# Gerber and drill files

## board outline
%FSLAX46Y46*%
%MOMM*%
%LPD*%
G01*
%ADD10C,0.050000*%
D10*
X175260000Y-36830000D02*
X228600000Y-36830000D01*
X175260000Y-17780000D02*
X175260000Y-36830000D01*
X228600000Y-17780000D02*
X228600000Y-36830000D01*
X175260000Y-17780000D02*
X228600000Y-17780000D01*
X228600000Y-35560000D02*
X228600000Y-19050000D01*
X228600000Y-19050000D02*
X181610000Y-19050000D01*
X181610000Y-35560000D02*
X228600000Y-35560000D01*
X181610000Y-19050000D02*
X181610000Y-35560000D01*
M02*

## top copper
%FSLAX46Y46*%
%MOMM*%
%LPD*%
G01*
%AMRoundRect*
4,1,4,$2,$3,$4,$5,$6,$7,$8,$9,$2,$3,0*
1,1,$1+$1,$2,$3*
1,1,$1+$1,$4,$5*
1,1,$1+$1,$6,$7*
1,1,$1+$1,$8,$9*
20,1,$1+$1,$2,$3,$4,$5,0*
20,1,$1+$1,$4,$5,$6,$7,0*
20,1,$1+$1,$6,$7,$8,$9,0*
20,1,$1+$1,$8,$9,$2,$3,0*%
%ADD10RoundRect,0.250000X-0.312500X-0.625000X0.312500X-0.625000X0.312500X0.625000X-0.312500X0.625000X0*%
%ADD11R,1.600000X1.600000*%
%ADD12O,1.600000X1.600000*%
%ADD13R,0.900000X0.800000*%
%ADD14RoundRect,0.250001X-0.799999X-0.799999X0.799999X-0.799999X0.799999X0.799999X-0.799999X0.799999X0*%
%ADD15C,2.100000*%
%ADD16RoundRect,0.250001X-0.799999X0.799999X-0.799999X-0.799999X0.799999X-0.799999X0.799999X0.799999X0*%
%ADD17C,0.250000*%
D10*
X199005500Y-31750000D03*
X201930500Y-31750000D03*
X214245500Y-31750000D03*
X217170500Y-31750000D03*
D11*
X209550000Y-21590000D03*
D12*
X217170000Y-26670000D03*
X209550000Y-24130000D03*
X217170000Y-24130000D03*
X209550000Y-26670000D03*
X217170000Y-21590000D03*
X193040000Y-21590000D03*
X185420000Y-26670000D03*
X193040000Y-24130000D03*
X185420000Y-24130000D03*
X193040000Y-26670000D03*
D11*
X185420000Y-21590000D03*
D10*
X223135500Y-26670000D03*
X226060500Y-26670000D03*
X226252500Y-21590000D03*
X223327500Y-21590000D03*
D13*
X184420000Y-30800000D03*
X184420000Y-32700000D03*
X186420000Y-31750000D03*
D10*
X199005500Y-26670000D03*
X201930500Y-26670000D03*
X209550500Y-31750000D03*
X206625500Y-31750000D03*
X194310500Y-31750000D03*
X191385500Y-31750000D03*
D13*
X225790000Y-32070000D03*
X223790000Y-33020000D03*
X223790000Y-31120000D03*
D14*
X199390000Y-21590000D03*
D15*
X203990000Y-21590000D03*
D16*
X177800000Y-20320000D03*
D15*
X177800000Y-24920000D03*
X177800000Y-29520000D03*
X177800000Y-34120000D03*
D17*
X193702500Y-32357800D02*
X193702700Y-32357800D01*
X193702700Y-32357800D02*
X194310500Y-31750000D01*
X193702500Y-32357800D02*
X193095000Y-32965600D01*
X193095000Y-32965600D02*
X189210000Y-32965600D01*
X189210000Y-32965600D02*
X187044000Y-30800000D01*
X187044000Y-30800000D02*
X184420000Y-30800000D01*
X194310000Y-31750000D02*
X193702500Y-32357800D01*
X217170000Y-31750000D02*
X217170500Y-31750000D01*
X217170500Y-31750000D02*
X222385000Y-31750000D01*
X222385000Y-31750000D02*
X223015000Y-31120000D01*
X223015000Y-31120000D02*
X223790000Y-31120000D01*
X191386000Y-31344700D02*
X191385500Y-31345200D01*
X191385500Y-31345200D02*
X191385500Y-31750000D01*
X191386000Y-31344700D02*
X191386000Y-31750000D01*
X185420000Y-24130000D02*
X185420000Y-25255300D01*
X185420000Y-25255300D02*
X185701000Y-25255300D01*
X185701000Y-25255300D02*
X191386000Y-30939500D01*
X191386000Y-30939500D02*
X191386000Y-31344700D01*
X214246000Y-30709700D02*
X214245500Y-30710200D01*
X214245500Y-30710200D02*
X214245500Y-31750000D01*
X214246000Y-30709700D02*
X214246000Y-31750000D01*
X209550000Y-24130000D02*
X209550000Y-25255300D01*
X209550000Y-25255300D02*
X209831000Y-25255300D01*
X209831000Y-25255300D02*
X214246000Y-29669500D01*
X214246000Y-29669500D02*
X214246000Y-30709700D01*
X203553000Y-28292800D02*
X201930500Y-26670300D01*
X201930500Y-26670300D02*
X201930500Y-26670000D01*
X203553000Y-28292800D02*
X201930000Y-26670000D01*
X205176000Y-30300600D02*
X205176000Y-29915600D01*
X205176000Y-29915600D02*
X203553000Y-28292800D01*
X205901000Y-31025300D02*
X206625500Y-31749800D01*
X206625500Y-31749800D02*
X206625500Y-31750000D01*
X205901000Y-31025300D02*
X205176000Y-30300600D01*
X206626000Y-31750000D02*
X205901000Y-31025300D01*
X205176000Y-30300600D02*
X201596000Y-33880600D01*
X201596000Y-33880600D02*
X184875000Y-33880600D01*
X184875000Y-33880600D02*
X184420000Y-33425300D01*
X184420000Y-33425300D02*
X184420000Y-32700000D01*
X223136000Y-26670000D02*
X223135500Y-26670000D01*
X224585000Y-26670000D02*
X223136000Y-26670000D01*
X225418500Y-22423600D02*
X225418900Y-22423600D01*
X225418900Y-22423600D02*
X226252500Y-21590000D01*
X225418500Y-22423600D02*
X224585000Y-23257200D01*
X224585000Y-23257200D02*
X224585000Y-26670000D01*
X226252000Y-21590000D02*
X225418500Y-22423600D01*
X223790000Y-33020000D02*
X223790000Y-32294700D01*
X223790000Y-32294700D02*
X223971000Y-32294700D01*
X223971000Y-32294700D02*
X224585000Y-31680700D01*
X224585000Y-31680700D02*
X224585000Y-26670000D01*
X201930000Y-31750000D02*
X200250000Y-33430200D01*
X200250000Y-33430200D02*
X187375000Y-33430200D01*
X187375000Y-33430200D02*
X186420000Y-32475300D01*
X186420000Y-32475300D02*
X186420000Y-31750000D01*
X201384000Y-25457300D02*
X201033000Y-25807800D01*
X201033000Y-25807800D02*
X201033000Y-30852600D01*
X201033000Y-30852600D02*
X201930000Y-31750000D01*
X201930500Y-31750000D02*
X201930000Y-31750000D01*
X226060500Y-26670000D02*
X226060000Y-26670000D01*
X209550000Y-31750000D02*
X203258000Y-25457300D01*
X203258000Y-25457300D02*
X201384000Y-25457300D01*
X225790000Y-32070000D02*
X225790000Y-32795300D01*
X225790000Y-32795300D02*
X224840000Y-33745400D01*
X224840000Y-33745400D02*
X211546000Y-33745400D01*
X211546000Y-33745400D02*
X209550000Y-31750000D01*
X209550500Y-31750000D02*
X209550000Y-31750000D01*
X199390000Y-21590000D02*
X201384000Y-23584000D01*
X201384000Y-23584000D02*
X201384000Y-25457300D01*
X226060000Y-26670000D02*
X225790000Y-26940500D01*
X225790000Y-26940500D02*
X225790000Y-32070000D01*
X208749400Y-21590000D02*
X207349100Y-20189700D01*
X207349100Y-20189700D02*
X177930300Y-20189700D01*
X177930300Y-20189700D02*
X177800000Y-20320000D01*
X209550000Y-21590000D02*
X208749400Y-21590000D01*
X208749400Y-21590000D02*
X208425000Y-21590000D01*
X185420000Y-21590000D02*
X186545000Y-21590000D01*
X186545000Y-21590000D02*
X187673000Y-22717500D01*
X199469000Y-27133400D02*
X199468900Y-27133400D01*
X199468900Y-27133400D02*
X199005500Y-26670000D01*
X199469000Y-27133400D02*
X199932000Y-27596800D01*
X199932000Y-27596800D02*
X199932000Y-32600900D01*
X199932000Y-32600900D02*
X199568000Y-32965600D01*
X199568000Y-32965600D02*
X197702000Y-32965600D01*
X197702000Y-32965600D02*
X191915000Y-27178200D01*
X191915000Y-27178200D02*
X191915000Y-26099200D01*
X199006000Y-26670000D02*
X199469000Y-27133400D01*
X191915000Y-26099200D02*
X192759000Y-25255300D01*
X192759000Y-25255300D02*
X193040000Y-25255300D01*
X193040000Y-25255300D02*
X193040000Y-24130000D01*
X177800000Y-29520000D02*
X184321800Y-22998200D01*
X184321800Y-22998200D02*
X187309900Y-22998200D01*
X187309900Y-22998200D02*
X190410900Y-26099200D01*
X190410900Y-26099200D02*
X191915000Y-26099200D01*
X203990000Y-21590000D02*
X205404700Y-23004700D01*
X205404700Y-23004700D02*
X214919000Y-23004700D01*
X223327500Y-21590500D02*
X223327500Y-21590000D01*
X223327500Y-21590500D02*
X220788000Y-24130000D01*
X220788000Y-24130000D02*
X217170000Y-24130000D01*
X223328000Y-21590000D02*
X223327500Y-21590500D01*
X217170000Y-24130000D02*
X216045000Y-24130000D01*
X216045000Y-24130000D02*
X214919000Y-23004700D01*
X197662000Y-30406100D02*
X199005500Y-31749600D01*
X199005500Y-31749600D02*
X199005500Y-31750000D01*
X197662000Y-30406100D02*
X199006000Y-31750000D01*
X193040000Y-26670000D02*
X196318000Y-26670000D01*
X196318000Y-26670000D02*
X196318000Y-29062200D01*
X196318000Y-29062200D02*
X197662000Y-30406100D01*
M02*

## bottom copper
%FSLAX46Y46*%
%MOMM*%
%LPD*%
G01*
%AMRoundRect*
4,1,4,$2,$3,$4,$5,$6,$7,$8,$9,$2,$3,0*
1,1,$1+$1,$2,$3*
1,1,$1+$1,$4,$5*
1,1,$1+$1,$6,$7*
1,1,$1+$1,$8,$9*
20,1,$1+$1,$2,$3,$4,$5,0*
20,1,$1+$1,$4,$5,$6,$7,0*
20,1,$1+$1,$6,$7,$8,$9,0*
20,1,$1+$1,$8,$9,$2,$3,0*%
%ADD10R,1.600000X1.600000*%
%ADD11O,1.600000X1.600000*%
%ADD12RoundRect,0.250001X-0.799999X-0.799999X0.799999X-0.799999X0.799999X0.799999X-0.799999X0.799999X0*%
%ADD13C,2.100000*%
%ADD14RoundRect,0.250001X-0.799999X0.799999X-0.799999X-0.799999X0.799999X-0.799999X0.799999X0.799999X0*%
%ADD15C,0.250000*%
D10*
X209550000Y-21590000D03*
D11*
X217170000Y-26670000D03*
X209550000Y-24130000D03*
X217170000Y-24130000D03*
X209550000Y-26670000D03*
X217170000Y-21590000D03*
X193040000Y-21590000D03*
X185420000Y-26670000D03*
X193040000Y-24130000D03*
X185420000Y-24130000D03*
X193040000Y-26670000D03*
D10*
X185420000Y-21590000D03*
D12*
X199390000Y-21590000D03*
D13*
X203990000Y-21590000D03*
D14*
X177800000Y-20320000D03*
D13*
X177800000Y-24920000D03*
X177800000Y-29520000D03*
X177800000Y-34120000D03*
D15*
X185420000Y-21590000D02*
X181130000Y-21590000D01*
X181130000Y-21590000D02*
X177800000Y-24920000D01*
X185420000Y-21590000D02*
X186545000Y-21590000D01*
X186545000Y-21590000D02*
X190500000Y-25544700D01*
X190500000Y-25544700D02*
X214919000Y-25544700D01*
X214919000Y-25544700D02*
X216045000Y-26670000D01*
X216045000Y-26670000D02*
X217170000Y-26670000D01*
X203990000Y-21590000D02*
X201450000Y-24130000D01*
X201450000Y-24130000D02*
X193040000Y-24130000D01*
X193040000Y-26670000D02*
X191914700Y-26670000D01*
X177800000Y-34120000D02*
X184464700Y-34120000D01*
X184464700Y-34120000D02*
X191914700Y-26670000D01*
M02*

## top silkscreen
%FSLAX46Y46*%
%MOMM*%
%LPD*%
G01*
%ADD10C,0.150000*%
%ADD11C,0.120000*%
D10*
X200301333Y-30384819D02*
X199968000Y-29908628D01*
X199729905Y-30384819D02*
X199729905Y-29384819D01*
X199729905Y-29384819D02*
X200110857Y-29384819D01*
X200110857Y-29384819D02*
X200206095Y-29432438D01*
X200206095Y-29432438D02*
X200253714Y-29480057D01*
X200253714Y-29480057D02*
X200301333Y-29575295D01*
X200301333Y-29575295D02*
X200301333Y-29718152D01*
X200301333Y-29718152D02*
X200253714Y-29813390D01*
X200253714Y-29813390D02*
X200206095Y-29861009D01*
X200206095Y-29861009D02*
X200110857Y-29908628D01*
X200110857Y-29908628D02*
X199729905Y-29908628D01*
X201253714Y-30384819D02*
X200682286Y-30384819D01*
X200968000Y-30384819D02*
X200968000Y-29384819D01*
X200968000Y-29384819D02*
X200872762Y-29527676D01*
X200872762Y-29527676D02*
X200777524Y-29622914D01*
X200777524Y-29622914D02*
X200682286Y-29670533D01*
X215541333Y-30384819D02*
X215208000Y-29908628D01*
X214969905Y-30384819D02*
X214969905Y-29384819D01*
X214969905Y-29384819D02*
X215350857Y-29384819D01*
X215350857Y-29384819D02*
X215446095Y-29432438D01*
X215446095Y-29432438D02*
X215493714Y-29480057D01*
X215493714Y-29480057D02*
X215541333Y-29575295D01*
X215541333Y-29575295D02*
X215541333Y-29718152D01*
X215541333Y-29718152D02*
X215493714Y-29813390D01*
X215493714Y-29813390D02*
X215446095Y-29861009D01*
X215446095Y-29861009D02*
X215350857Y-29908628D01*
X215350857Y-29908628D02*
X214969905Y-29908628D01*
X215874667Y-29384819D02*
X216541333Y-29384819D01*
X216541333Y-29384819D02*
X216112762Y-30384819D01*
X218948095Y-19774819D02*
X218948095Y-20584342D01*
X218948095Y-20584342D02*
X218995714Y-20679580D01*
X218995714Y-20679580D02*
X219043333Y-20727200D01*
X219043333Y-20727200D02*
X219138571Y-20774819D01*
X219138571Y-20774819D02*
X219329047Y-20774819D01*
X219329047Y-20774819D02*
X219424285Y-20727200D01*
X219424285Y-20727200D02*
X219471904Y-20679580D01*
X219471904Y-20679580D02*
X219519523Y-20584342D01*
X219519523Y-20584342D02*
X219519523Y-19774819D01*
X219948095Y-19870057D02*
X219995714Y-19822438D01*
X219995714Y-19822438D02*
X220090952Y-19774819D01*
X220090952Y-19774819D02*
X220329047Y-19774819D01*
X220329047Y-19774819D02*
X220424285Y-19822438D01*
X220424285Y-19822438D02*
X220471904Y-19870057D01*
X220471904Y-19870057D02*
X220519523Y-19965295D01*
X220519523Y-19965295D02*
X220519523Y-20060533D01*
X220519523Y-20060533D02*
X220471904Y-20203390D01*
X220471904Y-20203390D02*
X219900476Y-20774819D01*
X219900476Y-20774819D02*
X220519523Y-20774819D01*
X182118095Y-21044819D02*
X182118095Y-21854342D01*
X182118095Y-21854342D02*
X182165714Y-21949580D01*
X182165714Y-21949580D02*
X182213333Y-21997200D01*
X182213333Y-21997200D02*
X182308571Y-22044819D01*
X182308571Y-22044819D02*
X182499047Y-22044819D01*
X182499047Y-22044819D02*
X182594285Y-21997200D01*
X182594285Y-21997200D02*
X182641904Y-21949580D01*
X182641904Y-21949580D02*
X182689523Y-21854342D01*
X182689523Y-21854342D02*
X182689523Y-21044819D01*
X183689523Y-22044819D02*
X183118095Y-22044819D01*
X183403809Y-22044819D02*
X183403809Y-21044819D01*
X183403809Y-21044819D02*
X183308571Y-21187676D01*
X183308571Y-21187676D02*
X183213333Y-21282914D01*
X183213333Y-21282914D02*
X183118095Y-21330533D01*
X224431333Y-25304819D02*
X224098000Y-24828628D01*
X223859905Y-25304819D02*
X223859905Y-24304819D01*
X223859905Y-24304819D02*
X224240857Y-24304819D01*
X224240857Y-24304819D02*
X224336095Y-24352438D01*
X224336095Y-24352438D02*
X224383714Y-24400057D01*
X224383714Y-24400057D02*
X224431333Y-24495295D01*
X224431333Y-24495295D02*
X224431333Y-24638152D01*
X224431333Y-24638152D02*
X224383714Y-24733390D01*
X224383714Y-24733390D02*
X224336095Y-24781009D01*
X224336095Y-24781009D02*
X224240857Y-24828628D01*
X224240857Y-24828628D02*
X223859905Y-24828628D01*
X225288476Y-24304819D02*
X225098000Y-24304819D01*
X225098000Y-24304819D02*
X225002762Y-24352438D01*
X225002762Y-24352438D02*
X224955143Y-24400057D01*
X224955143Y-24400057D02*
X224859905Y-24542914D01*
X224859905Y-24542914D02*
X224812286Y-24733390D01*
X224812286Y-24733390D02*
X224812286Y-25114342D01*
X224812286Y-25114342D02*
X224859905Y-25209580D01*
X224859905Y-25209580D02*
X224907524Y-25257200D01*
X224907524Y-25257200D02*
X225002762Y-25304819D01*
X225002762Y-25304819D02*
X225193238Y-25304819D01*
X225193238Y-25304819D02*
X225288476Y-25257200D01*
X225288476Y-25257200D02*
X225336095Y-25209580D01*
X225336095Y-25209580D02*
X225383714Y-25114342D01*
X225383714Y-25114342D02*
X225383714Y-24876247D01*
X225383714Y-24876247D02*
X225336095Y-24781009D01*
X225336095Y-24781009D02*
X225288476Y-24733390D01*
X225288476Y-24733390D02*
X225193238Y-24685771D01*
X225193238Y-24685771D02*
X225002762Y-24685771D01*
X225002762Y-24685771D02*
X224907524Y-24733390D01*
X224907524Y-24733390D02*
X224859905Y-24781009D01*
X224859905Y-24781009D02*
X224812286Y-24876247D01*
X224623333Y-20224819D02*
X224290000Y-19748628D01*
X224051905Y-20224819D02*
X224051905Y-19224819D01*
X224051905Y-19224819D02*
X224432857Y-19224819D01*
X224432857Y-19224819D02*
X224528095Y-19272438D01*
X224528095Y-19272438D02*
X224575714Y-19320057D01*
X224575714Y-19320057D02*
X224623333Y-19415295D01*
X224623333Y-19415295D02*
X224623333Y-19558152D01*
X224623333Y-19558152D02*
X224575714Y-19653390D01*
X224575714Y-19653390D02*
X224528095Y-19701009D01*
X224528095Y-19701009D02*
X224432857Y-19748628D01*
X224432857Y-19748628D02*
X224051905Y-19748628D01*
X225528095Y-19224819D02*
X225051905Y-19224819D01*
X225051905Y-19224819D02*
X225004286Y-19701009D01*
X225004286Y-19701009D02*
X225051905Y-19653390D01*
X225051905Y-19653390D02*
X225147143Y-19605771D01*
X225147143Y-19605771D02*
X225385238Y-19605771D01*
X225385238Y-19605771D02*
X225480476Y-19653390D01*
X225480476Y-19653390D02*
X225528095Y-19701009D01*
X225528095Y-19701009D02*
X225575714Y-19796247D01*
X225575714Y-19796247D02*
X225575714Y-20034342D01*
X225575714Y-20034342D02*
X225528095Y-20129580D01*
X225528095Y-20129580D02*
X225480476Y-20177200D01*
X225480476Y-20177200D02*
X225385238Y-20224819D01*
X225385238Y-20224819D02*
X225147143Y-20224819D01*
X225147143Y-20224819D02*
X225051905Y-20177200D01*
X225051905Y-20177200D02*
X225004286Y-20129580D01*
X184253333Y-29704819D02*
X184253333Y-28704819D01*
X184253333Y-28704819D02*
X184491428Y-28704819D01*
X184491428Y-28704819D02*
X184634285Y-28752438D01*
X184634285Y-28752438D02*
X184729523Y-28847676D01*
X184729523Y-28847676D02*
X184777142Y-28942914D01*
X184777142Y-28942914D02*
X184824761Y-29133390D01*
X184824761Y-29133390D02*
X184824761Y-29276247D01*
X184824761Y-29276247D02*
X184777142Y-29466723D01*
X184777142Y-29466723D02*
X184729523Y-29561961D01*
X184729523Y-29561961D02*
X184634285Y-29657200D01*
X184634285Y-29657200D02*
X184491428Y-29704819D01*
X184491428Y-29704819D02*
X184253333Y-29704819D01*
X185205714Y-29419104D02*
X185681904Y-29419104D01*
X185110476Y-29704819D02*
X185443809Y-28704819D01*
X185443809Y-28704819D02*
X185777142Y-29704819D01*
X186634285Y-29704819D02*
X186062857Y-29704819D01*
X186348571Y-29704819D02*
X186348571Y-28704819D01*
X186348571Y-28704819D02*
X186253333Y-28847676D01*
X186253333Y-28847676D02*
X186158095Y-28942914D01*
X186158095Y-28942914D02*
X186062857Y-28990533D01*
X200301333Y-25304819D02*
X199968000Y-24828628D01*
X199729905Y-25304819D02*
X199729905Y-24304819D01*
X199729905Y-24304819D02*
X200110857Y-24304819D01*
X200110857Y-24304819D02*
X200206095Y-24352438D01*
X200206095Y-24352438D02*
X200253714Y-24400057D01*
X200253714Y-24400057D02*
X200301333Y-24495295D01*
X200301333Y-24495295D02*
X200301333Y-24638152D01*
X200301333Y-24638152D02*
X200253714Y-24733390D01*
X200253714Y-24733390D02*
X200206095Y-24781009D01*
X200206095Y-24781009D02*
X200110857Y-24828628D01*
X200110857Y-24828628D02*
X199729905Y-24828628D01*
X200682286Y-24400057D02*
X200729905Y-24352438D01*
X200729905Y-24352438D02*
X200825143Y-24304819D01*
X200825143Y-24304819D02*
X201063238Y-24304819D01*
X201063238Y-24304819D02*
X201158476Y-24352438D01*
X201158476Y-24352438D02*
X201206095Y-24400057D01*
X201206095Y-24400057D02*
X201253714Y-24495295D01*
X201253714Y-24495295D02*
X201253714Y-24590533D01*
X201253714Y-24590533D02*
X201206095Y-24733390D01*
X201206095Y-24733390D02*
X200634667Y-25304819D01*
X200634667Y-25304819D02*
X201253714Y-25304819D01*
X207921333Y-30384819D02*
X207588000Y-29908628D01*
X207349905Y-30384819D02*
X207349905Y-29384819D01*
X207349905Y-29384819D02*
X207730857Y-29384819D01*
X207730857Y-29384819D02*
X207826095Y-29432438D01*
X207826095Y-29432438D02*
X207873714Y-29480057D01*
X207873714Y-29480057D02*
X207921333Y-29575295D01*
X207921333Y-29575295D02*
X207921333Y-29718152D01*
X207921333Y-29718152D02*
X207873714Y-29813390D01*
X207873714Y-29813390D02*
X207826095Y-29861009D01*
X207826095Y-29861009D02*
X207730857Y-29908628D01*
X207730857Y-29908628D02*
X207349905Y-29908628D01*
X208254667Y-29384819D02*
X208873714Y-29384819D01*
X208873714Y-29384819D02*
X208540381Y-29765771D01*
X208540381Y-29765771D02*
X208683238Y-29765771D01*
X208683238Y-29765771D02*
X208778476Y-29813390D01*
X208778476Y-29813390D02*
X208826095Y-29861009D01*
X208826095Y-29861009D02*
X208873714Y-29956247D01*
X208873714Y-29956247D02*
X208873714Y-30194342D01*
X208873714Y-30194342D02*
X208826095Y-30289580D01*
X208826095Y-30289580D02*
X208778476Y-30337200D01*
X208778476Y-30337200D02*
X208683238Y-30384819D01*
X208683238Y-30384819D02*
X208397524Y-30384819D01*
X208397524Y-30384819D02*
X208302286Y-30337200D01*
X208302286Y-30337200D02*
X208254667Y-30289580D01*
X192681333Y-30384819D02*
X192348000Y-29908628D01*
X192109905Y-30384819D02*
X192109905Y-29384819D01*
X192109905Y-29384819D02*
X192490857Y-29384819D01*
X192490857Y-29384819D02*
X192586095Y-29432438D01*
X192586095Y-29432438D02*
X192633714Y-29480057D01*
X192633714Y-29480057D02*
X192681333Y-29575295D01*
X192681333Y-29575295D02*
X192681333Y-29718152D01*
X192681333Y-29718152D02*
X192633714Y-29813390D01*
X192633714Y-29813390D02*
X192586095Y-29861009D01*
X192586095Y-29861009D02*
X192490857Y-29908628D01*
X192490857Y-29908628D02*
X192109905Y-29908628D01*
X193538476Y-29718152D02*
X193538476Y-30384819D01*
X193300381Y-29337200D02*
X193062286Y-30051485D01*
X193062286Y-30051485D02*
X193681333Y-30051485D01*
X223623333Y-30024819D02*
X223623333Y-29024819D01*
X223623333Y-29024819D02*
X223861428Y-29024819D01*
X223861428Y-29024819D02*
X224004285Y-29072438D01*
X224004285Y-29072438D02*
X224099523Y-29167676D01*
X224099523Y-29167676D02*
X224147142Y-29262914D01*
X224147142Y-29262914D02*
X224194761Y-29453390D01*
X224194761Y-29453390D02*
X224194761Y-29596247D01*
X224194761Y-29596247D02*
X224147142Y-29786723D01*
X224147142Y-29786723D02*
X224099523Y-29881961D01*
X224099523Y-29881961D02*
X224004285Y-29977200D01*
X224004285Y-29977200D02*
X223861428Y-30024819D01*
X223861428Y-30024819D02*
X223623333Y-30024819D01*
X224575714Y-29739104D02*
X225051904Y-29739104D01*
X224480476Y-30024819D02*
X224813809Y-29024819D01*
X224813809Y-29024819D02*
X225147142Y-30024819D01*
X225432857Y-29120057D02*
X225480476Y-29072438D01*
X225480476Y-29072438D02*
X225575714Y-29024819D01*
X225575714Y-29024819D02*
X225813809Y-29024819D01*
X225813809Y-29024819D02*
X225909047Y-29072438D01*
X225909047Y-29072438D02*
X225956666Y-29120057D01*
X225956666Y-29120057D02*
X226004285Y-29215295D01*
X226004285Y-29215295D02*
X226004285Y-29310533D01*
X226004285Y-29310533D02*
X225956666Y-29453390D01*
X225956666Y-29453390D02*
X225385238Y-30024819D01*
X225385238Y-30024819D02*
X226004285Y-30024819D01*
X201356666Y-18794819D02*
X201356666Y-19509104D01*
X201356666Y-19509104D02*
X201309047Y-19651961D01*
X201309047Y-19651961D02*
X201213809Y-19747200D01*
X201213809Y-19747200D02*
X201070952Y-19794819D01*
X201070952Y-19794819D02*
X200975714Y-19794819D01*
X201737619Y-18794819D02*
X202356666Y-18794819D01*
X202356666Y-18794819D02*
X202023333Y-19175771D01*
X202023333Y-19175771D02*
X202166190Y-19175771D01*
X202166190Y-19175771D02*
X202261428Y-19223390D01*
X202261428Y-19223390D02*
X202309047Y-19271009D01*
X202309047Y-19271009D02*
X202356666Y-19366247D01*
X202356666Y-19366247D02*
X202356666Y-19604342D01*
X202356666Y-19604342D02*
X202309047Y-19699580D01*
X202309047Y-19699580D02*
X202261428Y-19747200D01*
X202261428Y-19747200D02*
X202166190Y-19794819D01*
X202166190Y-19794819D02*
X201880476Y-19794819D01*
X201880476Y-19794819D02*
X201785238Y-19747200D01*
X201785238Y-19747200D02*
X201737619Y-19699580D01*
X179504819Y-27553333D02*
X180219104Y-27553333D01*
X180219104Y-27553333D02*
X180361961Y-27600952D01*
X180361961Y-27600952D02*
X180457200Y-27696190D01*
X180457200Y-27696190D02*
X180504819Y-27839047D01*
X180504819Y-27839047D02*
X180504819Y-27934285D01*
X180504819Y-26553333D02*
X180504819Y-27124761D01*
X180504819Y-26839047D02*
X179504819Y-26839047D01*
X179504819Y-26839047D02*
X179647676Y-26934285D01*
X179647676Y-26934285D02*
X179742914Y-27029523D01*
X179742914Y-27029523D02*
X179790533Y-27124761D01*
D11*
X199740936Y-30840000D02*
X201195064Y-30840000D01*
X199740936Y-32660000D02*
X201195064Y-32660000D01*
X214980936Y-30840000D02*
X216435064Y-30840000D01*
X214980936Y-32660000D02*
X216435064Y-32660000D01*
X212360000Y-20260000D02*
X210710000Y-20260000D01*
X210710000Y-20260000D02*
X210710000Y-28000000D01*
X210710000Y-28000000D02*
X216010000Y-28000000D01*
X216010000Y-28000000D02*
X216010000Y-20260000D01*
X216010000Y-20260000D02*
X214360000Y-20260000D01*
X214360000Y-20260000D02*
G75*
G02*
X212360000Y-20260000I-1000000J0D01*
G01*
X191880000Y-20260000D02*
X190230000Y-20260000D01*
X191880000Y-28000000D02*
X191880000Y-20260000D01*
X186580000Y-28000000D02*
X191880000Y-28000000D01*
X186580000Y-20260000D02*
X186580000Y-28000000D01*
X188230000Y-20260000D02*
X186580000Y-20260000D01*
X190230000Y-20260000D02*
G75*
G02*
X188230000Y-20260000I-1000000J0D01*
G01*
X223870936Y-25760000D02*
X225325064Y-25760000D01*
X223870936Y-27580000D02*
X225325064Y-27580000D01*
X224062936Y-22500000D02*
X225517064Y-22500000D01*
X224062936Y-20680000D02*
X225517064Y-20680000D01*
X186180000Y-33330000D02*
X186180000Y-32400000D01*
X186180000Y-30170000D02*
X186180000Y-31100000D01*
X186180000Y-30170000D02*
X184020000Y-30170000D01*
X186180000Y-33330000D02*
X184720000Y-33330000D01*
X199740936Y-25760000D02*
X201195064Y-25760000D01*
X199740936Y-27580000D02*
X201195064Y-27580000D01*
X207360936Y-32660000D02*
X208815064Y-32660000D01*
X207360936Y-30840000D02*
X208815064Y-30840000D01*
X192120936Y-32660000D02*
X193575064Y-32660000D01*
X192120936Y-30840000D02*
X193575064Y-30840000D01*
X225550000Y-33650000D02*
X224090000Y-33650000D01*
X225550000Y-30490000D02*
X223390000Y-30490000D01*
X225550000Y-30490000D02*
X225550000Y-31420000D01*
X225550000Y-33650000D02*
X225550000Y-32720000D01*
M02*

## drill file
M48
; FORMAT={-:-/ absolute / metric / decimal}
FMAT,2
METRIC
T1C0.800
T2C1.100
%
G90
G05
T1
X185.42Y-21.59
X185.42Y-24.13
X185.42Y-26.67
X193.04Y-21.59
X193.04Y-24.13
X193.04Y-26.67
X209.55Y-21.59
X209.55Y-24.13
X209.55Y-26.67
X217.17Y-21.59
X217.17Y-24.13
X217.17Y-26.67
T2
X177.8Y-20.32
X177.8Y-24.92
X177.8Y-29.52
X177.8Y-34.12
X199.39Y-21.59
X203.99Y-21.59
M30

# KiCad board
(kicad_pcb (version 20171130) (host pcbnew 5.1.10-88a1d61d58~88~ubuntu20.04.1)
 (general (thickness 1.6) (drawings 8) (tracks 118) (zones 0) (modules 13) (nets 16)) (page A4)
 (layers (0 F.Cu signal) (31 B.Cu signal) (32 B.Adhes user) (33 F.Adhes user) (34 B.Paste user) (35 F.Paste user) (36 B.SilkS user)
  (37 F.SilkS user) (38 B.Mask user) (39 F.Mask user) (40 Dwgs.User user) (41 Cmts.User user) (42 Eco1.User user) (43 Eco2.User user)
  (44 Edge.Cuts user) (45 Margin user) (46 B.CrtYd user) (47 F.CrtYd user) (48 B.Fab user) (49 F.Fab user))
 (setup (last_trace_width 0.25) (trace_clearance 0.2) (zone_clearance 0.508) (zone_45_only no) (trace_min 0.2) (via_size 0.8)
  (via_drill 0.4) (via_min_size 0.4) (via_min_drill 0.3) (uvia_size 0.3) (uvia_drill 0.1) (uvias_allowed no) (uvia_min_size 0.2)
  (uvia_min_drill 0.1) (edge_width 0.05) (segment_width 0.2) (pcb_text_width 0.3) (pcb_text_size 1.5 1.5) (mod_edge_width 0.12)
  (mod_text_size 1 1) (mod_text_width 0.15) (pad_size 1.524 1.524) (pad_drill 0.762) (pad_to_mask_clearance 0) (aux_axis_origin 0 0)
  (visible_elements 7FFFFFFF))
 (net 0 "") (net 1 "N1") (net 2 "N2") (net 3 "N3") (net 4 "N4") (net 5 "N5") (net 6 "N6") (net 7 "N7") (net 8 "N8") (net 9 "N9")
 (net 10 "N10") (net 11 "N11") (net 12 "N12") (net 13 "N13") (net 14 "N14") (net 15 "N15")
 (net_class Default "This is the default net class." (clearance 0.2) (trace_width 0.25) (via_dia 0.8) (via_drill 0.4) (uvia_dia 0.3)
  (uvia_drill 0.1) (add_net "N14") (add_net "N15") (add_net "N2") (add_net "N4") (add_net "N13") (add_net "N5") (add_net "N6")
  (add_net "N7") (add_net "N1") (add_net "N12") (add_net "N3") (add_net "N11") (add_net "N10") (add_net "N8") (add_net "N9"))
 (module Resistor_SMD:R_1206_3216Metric (layer F.Cu) (at 200.468 31.75)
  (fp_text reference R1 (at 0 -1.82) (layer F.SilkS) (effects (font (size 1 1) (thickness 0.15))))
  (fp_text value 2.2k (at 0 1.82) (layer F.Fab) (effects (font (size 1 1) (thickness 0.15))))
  (fp_line (start -0.727064 -0.91) (end 0.727064 -0.91) (layer F.SilkS) (width 0.12))
  (fp_line (start -0.727064 0.91) (end 0.727064 0.91) (layer F.SilkS) (width 0.12))
  (pad 1 smd roundrect (at -1.4625 0) (size 1.125 1.75) (layers F.Cu F.Paste F.Mask) (roundrect_rratio 0.222222) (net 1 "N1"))
  (pad 2 smd roundrect (at 1.4625 0) (size 1.125 1.75) (layers F.Cu F.Paste F.Mask) (roundrect_rratio 0.222222) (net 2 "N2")))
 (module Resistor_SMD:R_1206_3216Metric (layer F.Cu) (at 215.708 31.75)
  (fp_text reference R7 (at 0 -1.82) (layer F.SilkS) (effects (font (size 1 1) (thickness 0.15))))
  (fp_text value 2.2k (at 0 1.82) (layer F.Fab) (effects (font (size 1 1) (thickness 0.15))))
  (fp_line (start -0.727064 -0.91) (end 0.727064 -0.91) (layer F.SilkS) (width 0.12))
  (fp_line (start -0.727064 0.91) (end 0.727064 0.91) (layer F.SilkS) (width 0.12))
  (pad 1 smd roundrect (at -1.4625 0) (size 1.125 1.75) (layers F.Cu F.Paste F.Mask) (roundrect_rratio 0.222222) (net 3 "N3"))
  (pad 2 smd roundrect (at 1.4625 0) (size 1.125 1.75) (layers F.Cu F.Paste F.Mask) (roundrect_rratio 0.222222) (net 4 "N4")))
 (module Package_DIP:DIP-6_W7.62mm (layer F.Cu) (at 209.55 21.59)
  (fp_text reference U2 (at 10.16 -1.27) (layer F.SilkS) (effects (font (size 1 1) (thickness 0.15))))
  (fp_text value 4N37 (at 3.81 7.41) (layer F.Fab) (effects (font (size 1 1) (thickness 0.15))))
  (fp_line (start 2.81 -1.33) (end 1.16 -1.33) (layer F.SilkS) (width 0.12))
  (fp_line (start 1.16 -1.33) (end 1.16 6.41) (layer F.SilkS) (width 0.12))
  (fp_line (start 1.16 6.41) (end 6.46 6.41) (layer F.SilkS) (width 0.12))
  (fp_line (start 6.46 6.41) (end 6.46 -1.33) (layer F.SilkS) (width 0.12))
  (fp_line (start 6.46 -1.33) (end 4.81 -1.33) (layer F.SilkS) (width 0.12))
  (fp_arc (start 3.81 -1.33) (end 2.81 -1.33) (angle -180) (layer F.SilkS) (width 0.12))
  (pad 1 thru_hole rect (at 0 0) (size 1.6 1.6) (drill 0.8) (layers *.Cu *.Mask) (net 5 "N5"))
  (pad 4 thru_hole oval (at 7.62 5.08) (size 1.6 1.6) (drill 0.8) (layers *.Cu *.Mask) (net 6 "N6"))
  (pad 2 thru_hole oval (at 0 2.54) (size 1.6 1.6) (drill 0.8) (layers *.Cu *.Mask) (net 3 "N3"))
  (pad 5 thru_hole oval (at 7.62 2.54) (size 1.6 1.6) (drill 0.8) (layers *.Cu *.Mask) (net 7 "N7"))
  (pad 3 thru_hole oval (at 0 5.08) (size 1.6 1.6) (drill 0.8) (layers *.Cu *.Mask) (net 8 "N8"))
  (pad 6 thru_hole oval (at 7.62 0) (size 1.6 1.6) (drill 0.8) (layers *.Cu *.Mask) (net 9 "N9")))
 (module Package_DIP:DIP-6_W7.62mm (layer F.Cu) (at 185.42 21.59)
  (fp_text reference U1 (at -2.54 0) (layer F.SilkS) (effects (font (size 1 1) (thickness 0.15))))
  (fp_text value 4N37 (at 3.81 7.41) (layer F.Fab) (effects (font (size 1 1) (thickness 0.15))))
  (fp_line (start 6.46 -1.33) (end 4.81 -1.33) (layer F.SilkS) (width 0.12))
  (fp_line (start 6.46 6.41) (end 6.46 -1.33) (layer F.SilkS) (width 0.12))
  (fp_line (start 1.16 6.41) (end 6.46 6.41) (layer F.SilkS) (width 0.12))
  (fp_line (start 1.16 -1.33) (end 1.16 6.41) (layer F.SilkS) (width 0.12))
  (fp_line (start 2.81 -1.33) (end 1.16 -1.33) (layer F.SilkS) (width 0.12))
  (fp_arc (start 3.81 -1.33) (end 2.81 -1.33) (angle -180) (layer F.SilkS) (width 0.12))
  (pad 6 thru_hole oval (at 7.62 0) (size 1.6 1.6) (drill 0.8) (layers *.Cu *.Mask) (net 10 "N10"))
  (pad 3 thru_hole oval (at 0 5.08) (size 1.6 1.6) (drill 0.8) (layers *.Cu *.Mask) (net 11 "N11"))
  (pad 5 thru_hole oval (at 7.62 2.54) (size 1.6 1.6) (drill 0.8) (layers *.Cu *.Mask) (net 7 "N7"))
  (pad 2 thru_hole oval (at 0 2.54) (size 1.6 1.6) (drill 0.8) (layers *.Cu *.Mask) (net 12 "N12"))
  (pad 4 thru_hole oval (at 7.62 5.08) (size 1.6 1.6) (drill 0.8) (layers *.Cu *.Mask) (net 1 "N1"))
  (pad 1 thru_hole rect (at 0 0) (size 1.6 1.6) (drill 0.8) (layers *.Cu *.Mask) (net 6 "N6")))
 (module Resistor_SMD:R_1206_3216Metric (layer F.Cu) (at 224.598 26.67)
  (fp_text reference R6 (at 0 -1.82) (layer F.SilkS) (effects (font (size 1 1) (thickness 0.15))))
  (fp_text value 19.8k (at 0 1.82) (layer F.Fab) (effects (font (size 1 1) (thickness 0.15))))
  (fp_line (start -0.727064 -0.91) (end 0.727064 -0.91) (layer F.SilkS) (width 0.12))
  (fp_line (start -0.727064 0.91) (end 0.727064 0.91) (layer F.SilkS) (width 0.12))
  (pad 1 smd roundrect (at -1.4625 0) (size 1.125 1.75) (layers F.Cu F.Paste F.Mask) (roundrect_rratio 0.222222) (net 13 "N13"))
  (pad 2 smd roundrect (at 1.4625 0) (size 1.125 1.75) (layers F.Cu F.Paste F.Mask) (roundrect_rratio 0.222222) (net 2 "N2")))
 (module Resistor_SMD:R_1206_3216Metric (layer F.Cu) (at 224.79 21.59)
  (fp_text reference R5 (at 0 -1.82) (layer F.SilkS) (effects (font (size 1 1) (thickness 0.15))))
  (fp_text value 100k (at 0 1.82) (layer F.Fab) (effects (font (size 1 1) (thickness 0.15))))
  (fp_line (start -0.727064 0.91) (end 0.727064 0.91) (layer F.SilkS) (width 0.12))
  (fp_line (start -0.727064 -0.91) (end 0.727064 -0.91) (layer F.SilkS) (width 0.12))
  (pad 2 smd roundrect (at 1.4625 0) (size 1.125 1.75) (layers F.Cu F.Paste F.Mask) (roundrect_rratio 0.222222) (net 13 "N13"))
  (pad 1 smd roundrect (at -1.4625 0) (size 1.125 1.75) (layers F.Cu F.Paste F.Mask) (roundrect_rratio 0.222222) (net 7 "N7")))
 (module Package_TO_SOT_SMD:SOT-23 (layer F.Cu) (at 185.42 31.75)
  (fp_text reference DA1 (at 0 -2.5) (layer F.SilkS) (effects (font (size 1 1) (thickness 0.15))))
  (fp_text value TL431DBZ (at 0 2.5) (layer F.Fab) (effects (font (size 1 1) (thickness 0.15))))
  (fp_line (start 0.76 1.58) (end 0.76 0.65) (layer F.SilkS) (width 0.12))
  (fp_line (start 0.76 -1.58) (end 0.76 -0.65) (layer F.SilkS) (width 0.12))
  (fp_line (start 0.76 -1.58) (end -1.4 -1.58) (layer F.SilkS) (width 0.12))
  (fp_line (start 0.76 1.58) (end -0.7 1.58) (layer F.SilkS) (width 0.12))
  (pad 1 smd rect (at -1 -0.95) (size 0.9 0.8) (layers F.Cu F.Paste F.Mask) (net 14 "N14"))
  (pad 2 smd rect (at -1 0.95) (size 0.9 0.8) (layers F.Cu F.Paste F.Mask) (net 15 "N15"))
  (pad 3 smd rect (at 1 0) (size 0.9 0.8) (layers F.Cu F.Paste F.Mask) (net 2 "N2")))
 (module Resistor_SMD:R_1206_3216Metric (layer F.Cu) (at 200.468 26.67)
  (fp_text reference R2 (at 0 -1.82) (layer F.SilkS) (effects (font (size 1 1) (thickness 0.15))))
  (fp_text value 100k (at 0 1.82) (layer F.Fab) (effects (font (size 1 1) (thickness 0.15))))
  (fp_line (start -0.727064 -0.91) (end 0.727064 -0.91) (layer F.SilkS) (width 0.12))
  (fp_line (start -0.727064 0.91) (end 0.727064 0.91) (layer F.SilkS) (width 0.12))
  (pad 1 smd roundrect (at -1.4625 0) (size 1.125 1.75) (layers F.Cu F.Paste F.Mask) (roundrect_rratio 0.222222) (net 7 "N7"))
  (pad 2 smd roundrect (at 1.4625 0) (size 1.125 1.75) (layers F.Cu F.Paste F.Mask) (roundrect_rratio 0.222222) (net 15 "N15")))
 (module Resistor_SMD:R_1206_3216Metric (layer F.Cu) (at 208.088 31.75)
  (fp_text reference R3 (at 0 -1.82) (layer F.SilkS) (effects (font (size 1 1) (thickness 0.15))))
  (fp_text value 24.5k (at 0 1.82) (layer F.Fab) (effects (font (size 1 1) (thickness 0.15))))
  (fp_line (start -0.727064 0.91) (end 0.727064 0.91) (layer F.SilkS) (width 0.12))
  (fp_line (start -0.727064 -0.91) (end 0.727064 -0.91) (layer F.SilkS) (width 0.12))
  (pad 2 smd roundrect (at 1.4625 0) (size 1.125 1.75) (layers F.Cu F.Paste F.Mask) (roundrect_rratio 0.222222) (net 2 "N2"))
  (pad 1 smd roundrect (at -1.4625 0) (size 1.125 1.75) (layers F.Cu F.Paste F.Mask) (roundrect_rratio 0.222222) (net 15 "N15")))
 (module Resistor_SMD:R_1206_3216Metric (layer F.Cu) (at 192.848 31.75)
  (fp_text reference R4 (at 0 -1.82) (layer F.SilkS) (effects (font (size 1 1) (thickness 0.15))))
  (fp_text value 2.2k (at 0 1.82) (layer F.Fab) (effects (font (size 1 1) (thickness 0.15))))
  (fp_line (start -0.727064 0.91) (end 0.727064 0.91) (layer F.SilkS) (width 0.12))
  (fp_line (start -0.727064 -0.91) (end 0.727064 -0.91) (layer F.SilkS) (width 0.12))
  (pad 2 smd roundrect (at 1.4625 0) (size 1.125 1.75) (layers F.Cu F.Paste F.Mask) (roundrect_rratio 0.222222) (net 14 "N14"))
  (pad 1 smd roundrect (at -1.4625 0) (size 1.125 1.75) (layers F.Cu F.Paste F.Mask) (roundrect_rratio 0.222222) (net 12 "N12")))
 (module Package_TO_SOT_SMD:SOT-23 (layer F.Cu) (at 224.79 32.07)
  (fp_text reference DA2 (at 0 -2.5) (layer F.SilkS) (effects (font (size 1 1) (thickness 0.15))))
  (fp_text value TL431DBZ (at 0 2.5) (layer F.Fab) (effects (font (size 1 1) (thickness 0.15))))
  (fp_line (start 0.76 1.58) (end -0.7 1.58) (layer F.SilkS) (width 0.12))
  (fp_line (start 0.76 -1.58) (end -1.4 -1.58) (layer F.SilkS) (width 0.12))
  (fp_line (start 0.76 -1.58) (end 0.76 -0.65) (layer F.SilkS) (width 0.12))
  (fp_line (start 0.76 1.58) (end 0.76 0.65) (layer F.SilkS) (width 0.12))
  (pad 3 smd rect (at 1 0) (size 0.9 0.8) (layers F.Cu F.Paste F.Mask) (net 2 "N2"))
  (pad 2 smd rect (at -1 0.95) (size 0.9 0.8) (layers F.Cu F.Paste F.Mask) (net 13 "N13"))
  (pad 1 smd rect (at -1 -0.95) (size 0.9 0.8) (layers F.Cu F.Paste F.Mask) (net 4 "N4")))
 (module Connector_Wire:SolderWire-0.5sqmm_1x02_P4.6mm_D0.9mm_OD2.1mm (layer F.Cu) (at 199.39 21.59)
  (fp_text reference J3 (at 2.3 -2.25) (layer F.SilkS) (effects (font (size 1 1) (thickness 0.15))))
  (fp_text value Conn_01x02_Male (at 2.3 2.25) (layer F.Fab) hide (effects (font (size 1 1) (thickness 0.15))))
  (pad 1 thru_hole roundrect (at 0 0) (size 2.1 2.1) (drill 1.1) (layers *.Cu *.Mask) (roundrect_rratio 0.119048) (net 2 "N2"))
  (pad 2 thru_hole circle (at 4.6 0) (size 2.1 2.1) (drill 1.1) (layers *.Cu *.Mask) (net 7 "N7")))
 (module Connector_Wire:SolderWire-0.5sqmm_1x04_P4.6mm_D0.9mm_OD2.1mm (layer F.Cu) (at 177.8 20.32 270)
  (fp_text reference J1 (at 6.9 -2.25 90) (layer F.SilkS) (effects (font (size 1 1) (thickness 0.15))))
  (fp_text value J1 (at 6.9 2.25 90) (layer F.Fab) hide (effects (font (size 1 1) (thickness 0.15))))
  (pad 1 thru_hole roundrect (at 0 0 270) (size 2.1 2.1) (drill 1.1) (layers *.Cu *.Mask) (roundrect_rratio 0.119048) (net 5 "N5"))
  (pad 2 thru_hole circle (at 4.6 0 270) (size 2.1 2.1) (drill 1.1) (layers *.Cu *.Mask) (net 6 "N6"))
  (pad 3 thru_hole circle (at 9.2 0 270) (size 2.1 2.1) (drill 1.1) (layers *.Cu *.Mask) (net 7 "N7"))
  (pad 4 thru_hole circle (at 13.8 0 270) (size 2.1 2.1) (drill 1.1) (layers *.Cu *.Mask) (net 1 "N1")))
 (gr_line (start 175.26 36.83) (end 228.6 36.83) (layer Edge.Cuts) (width 0.05))
 (gr_line (start 175.26 17.78) (end 175.26 36.83) (layer Edge.Cuts) (width 0.05))
 (gr_line (start 228.6 17.78) (end 228.6 36.83) (layer Edge.Cuts) (width 0.05))
 (gr_line (start 175.26 17.78) (end 228.6 17.78) (layer Edge.Cuts) (width 0.05))
 (gr_line (start 228.6 35.56) (end 228.6 19.05) (layer Edge.Cuts) (width 0.05))
 (gr_line (start 228.6 19.05) (end 181.61 19.05) (layer Edge.Cuts) (width 0.05))
 (gr_line (start 181.61 35.56) (end 228.6 35.56) (layer Edge.Cuts) (width 0.05))
 (gr_line (start 181.61 19.05) (end 181.61 35.56) (layer Edge.Cuts) (width 0.05))
 (segment (start 193.7025 32.3578) (end 193.7027 32.3578) (width 0.25) (layer F.Cu) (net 14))
 (segment (start 193.7027 32.3578) (end 194.3105 31.75) (width 0.25) (layer F.Cu) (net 14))
 (segment (start 193.7025 32.3578) (end 193.095 32.9656) (width 0.25) (layer F.Cu) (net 14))
 (segment (start 193.095 32.9656) (end 189.21 32.9656) (width 0.25) (layer F.Cu) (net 14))
 (segment (start 189.21 32.9656) (end 187.044 30.8) (width 0.25) (layer F.Cu) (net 14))
 (segment (start 187.044 30.8) (end 184.42 30.8) (width 0.25) (layer F.Cu) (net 14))
 (segment (start 194.31 31.75) (end 193.7025 32.3578) (width 0.25) (layer F.Cu) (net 14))
 (segment (start 217.17 31.75) (end 217.1705 31.75) (width 0.25) (layer F.Cu) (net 4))
 (segment (start 217.1705 31.75) (end 222.385 31.75) (width 0.25) (layer F.Cu) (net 4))
 (segment (start 222.385 31.75) (end 223.015 31.12) (width 0.25) (layer F.Cu) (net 4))
 (segment (start 223.015 31.12) (end 223.79 31.12) (width 0.25) (layer F.Cu) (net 4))
 (segment (start 191.386 31.3447) (end 191.3855 31.3452) (width 0.25) (layer F.Cu) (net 12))
 (segment (start 191.3855 31.3452) (end 191.3855 31.75) (width 0.25) (layer F.Cu) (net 12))
 (segment (start 191.386 31.3447) (end 191.386 31.75) (width 0.25) (layer F.Cu) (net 12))
 (segment (start 185.42 24.13) (end 185.42 25.2553) (width 0.25) (layer F.Cu) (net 12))
 (segment (start 185.42 25.2553) (end 185.701 25.2553) (width 0.25) (layer F.Cu) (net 12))
 (segment (start 185.701 25.2553) (end 191.386 30.9395) (width 0.25) (layer F.Cu) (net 12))
 (segment (start 191.386 30.9395) (end 191.386 31.3447) (width 0.25) (layer F.Cu) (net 12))
 (segment (start 214.246 30.7097) (end 214.2455 30.7102) (width 0.25) (layer F.Cu) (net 3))
 (segment (start 214.2455 30.7102) (end 214.2455 31.75) (width 0.25) (layer F.Cu) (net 3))
 (segment (start 214.246 30.7097) (end 214.246 31.75) (width 0.25) (layer F.Cu) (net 3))
 (segment (start 209.55 24.13) (end 209.55 25.2553) (width 0.25) (layer F.Cu) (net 3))
 (segment (start 209.55 25.2553) (end 209.831 25.2553) (width 0.25) (layer F.Cu) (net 3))
 (segment (start 209.831 25.2553) (end 214.246 29.6695) (width 0.25) (layer F.Cu) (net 3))
 (segment (start 214.246 29.6695) (end 214.246 30.7097) (width 0.25) (layer F.Cu) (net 3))
 (segment (start 203.553 28.2928) (end 201.9305 26.6703) (width 0.25) (layer F.Cu) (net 15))
 (segment (start 201.9305 26.6703) (end 201.9305 26.67) (width 0.25) (layer F.Cu) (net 15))
 (segment (start 203.553 28.2928) (end 201.93 26.67) (width 0.25) (layer F.Cu) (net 15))
 (segment (start 205.176 30.3006) (end 205.176 29.9156) (width 0.25) (layer F.Cu) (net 15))
 (segment (start 205.176 29.9156) (end 203.553 28.2928) (width 0.25) (layer F.Cu) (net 15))
 (segment (start 205.901 31.0253) (end 206.6255 31.7498) (width 0.25) (layer F.Cu) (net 15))
 (segment (start 206.6255 31.7498) (end 206.6255 31.75) (width 0.25) (layer F.Cu) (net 15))
 (segment (start 205.901 31.0253) (end 205.176 30.3006) (width 0.25) (layer F.Cu) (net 15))
 (segment (start 206.626 31.75) (end 205.901 31.0253) (width 0.25) (layer F.Cu) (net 15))
 (segment (start 205.176 30.3006) (end 201.596 33.8806) (width 0.25) (layer F.Cu) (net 15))
 (segment (start 201.596 33.8806) (end 184.875 33.8806) (width 0.25) (layer F.Cu) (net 15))
 (segment (start 184.875 33.8806) (end 184.42 33.4253) (width 0.25) (layer F.Cu) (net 15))
 (segment (start 184.42 33.4253) (end 184.42 32.7) (width 0.25) (layer F.Cu) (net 15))
 (segment (start 223.136 26.67) (end 223.1355 26.67) (width 0.25) (layer F.Cu) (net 13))
 (segment (start 224.585 26.67) (end 223.136 26.67) (width 0.25) (layer F.Cu) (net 13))
 (segment (start 225.4185 22.4236) (end 225.4189 22.4236) (width 0.25) (layer F.Cu) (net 13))
 (segment (start 225.4189 22.4236) (end 226.2525 21.59) (width 0.25) (layer F.Cu) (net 13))
 (segment (start 225.4185 22.4236) (end 224.585 23.2572) (width 0.25) (layer F.Cu) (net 13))
 (segment (start 224.585 23.2572) (end 224.585 26.67) (width 0.25) (layer F.Cu) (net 13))
 (segment (start 226.252 21.59) (end 225.4185 22.4236) (width 0.25) (layer F.Cu) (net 13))
 (segment (start 223.79 33.02) (end 223.79 32.2947) (width 0.25) (layer F.Cu) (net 13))
 (segment (start 223.79 32.2947) (end 223.971 32.2947) (width 0.25) (layer F.Cu) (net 13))
 (segment (start 223.971 32.2947) (end 224.585 31.6807) (width 0.25) (layer F.Cu) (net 13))
 (segment (start 224.585 31.6807) (end 224.585 26.67) (width 0.25) (layer F.Cu) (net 13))
 (segment (start 201.93 31.75) (end 200.25 33.4302) (width 0.25) (layer F.Cu) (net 2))
 (segment (start 200.25 33.4302) (end 187.375 33.4302) (width 0.25) (layer F.Cu) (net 2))
 (segment (start 187.375 33.4302) (end 186.42 32.4753) (width 0.25) (layer F.Cu) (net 2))
 (segment (start 186.42 32.4753) (end 186.42 31.75) (width 0.25) (layer F.Cu) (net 2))
 (segment (start 201.384 25.4573) (end 201.033 25.8078) (width 0.25) (layer F.Cu) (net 2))
 (segment (start 201.033 25.8078) (end 201.033 30.8526) (width 0.25) (layer F.Cu) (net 2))
 (segment (start 201.033 30.8526) (end 201.93 31.75) (width 0.25) (layer F.Cu) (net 2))
 (segment (start 201.9305 31.75) (end 201.93 31.75) (width 0.25) (layer F.Cu) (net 2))
 (segment (start 226.0605 26.67) (end 226.06 26.67) (width 0.25) (layer F.Cu) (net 2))
 (segment (start 209.55 31.75) (end 203.258 25.4573) (width 0.25) (layer F.Cu) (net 2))
 (segment (start 203.258 25.4573) (end 201.384 25.4573) (width 0.25) (layer F.Cu) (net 2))
 (segment (start 225.79 32.07) (end 225.79 32.7953) (width 0.25) (layer F.Cu) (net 2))
 (segment (start 225.79 32.7953) (end 224.84 33.7454) (width 0.25) (layer F.Cu) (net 2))
 (segment (start 224.84 33.7454) (end 211.546 33.7454) (width 0.25) (layer F.Cu) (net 2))
 (segment (start 211.546 33.7454) (end 209.55 31.75) (width 0.25) (layer F.Cu) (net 2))
 (segment (start 209.5505 31.75) (end 209.55 31.75) (width 0.25) (layer F.Cu) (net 2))
 (segment (start 199.39 21.59) (end 201.384 23.584) (width 0.25) (layer F.Cu) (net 2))
 (segment (start 201.384 23.584) (end 201.384 25.4573) (width 0.25) (layer F.Cu) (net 2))
 (segment (start 226.06 26.67) (end 225.79 26.9405) (width 0.25) (layer F.Cu) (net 2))
 (segment (start 225.79 26.9405) (end 225.79 32.07) (width 0.25) (layer F.Cu) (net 2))
 (segment (start 208.7494 21.59) (end 207.3491 20.1897) (width 0.25) (layer F.Cu) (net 5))
 (segment (start 207.3491 20.1897) (end 177.9303 20.1897) (width 0.25) (layer F.Cu) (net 5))
 (segment (start 177.9303 20.1897) (end 177.8 20.32) (width 0.25) (layer F.Cu) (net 5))
 (segment (start 209.55 21.59) (end 208.7494 21.59) (width 0.25) (layer F.Cu) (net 5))
 (segment (start 208.7494 21.59) (end 208.425 21.59) (width 0.25) (layer F.Cu) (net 5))
 (segment (start 185.42 21.59) (end 181.13 21.59) (width 0.25) (layer B.Cu) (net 6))
 (segment (start 181.13 21.59) (end 177.8 24.92) (width 0.25) (layer B.Cu) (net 6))
 (segment (start 185.42 21.59) (end 186.545 21.59) (width 0.25) (layer B.Cu) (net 6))
 (segment (start 186.545 21.59) (end 190.5 25.5447) (width 0.25) (layer B.Cu) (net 6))
 (segment (start 190.5 25.5447) (end 214.919 25.5447) (width 0.25) (layer B.Cu) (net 6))
 (segment (start 214.919 25.5447) (end 216.045 26.67) (width 0.25) (layer B.Cu) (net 6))
 (segment (start 216.045 26.67) (end 217.17 26.67) (width 0.25) (layer B.Cu) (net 6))
 (segment (start 185.42 21.59) (end 186.545 21.59) (width 0.25) (layer F.Cu) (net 6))
 (segment (start 186.545 21.59) (end 187.673 22.7175) (width 0.25) (layer F.Cu) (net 6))
 (segment (start 199.469 27.1334) (end 199.4689 27.1334) (width 0.25) (layer F.Cu) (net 7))
 (segment (start 199.4689 27.1334) (end 199.0055 26.67) (width 0.25) (layer F.Cu) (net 7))
 (segment (start 199.469 27.1334) (end 199.932 27.5968) (width 0.25) (layer F.Cu) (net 7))
 (segment (start 199.932 27.5968) (end 199.932 32.6009) (width 0.25) (layer F.Cu) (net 7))
 (segment (start 199.932 32.6009) (end 199.568 32.9656) (width 0.25) (layer F.Cu) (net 7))
 (segment (start 199.568 32.9656) (end 197.702 32.9656) (width 0.25) (layer F.Cu) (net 7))
 (segment (start 197.702 32.9656) (end 191.915 27.1782) (width 0.25) (layer F.Cu) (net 7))
 (segment (start 191.915 27.1782) (end 191.915 26.0992) (width 0.25) (layer F.Cu) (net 7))
 (segment (start 199.006 26.67) (end 199.469 27.1334) (width 0.25) (layer F.Cu) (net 7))
 (segment (start 191.915 26.0992) (end 192.759 25.2553) (width 0.25) (layer F.Cu) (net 7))
 (segment (start 192.759 25.2553) (end 193.04 25.2553) (width 0.25) (layer F.Cu) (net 7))
 (segment (start 193.04 25.2553) (end 193.04 24.13) (width 0.25) (layer F.Cu) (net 7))
 (segment (start 177.8 29.52) (end 184.3218 22.9982) (width 0.25) (layer F.Cu) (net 7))
 (segment (start 184.3218 22.9982) (end 187.3099 22.9982) (width 0.25) (layer F.Cu) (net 7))
 (segment (start 187.3099 22.9982) (end 190.4109 26.0992) (width 0.25) (layer F.Cu) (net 7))
 (segment (start 190.4109 26.0992) (end 191.915 26.0992) (width 0.25) (layer F.Cu) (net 7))
 (segment (start 203.99 21.59) (end 201.45 24.13) (width 0.25) (layer B.Cu) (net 7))
 (segment (start 201.45 24.13) (end 193.04 24.13) (width 0.25) (layer B.Cu) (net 7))
 (segment (start 203.99 21.59) (end 205.4047 23.0047) (width 0.25) (layer F.Cu) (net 7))
 (segment (start 205.4047 23.0047) (end 214.919 23.0047) (width 0.25) (layer F.Cu) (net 7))
 (segment (start 223.3275 21.5905) (end 223.3275 21.59) (width 0.25) (layer F.Cu) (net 7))
 (segment (start 223.3275 21.5905) (end 220.788 24.13) (width 0.25) (layer F.Cu) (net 7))
 (segment (start 220.788 24.13) (end 217.17 24.13) (width 0.25) (layer F.Cu) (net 7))
 (segment (start 223.328 21.59) (end 223.3275 21.5905) (width 0.25) (layer F.Cu) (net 7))
 (segment (start 217.17 24.13) (end 216.045 24.13) (width 0.25) (layer F.Cu) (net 7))
 (segment (start 216.045 24.13) (end 214.919 23.0047) (width 0.25) (layer F.Cu) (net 7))
 (segment (start 193.04 26.67) (end 191.9147 26.67) (width 0.25) (layer B.Cu) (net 1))
 (segment (start 177.8 34.12) (end 184.4647 34.12) (width 0.25) (layer B.Cu) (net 1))
 (segment (start 184.4647 34.12) (end 191.9147 26.67) (width 0.25) (layer B.Cu) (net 1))
 (segment (start 197.662 30.4061) (end 199.0055 31.7496) (width 0.25) (layer F.Cu) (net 1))
 (segment (start 199.0055 31.7496) (end 199.0055 31.75) (width 0.25) (layer F.Cu) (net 1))
 (segment (start 197.662 30.4061) (end 199.006 31.75) (width 0.25) (layer F.Cu) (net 1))
 (segment (start 193.04 26.67) (end 196.318 26.67) (width 0.25) (layer F.Cu) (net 1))
 (segment (start 196.318 26.67) (end 196.318 29.0622) (width 0.25) (layer F.Cu) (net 1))
 (segment (start 196.318 29.0622) (end 197.662 30.4061) (width 0.25) (layer F.Cu) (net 1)))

